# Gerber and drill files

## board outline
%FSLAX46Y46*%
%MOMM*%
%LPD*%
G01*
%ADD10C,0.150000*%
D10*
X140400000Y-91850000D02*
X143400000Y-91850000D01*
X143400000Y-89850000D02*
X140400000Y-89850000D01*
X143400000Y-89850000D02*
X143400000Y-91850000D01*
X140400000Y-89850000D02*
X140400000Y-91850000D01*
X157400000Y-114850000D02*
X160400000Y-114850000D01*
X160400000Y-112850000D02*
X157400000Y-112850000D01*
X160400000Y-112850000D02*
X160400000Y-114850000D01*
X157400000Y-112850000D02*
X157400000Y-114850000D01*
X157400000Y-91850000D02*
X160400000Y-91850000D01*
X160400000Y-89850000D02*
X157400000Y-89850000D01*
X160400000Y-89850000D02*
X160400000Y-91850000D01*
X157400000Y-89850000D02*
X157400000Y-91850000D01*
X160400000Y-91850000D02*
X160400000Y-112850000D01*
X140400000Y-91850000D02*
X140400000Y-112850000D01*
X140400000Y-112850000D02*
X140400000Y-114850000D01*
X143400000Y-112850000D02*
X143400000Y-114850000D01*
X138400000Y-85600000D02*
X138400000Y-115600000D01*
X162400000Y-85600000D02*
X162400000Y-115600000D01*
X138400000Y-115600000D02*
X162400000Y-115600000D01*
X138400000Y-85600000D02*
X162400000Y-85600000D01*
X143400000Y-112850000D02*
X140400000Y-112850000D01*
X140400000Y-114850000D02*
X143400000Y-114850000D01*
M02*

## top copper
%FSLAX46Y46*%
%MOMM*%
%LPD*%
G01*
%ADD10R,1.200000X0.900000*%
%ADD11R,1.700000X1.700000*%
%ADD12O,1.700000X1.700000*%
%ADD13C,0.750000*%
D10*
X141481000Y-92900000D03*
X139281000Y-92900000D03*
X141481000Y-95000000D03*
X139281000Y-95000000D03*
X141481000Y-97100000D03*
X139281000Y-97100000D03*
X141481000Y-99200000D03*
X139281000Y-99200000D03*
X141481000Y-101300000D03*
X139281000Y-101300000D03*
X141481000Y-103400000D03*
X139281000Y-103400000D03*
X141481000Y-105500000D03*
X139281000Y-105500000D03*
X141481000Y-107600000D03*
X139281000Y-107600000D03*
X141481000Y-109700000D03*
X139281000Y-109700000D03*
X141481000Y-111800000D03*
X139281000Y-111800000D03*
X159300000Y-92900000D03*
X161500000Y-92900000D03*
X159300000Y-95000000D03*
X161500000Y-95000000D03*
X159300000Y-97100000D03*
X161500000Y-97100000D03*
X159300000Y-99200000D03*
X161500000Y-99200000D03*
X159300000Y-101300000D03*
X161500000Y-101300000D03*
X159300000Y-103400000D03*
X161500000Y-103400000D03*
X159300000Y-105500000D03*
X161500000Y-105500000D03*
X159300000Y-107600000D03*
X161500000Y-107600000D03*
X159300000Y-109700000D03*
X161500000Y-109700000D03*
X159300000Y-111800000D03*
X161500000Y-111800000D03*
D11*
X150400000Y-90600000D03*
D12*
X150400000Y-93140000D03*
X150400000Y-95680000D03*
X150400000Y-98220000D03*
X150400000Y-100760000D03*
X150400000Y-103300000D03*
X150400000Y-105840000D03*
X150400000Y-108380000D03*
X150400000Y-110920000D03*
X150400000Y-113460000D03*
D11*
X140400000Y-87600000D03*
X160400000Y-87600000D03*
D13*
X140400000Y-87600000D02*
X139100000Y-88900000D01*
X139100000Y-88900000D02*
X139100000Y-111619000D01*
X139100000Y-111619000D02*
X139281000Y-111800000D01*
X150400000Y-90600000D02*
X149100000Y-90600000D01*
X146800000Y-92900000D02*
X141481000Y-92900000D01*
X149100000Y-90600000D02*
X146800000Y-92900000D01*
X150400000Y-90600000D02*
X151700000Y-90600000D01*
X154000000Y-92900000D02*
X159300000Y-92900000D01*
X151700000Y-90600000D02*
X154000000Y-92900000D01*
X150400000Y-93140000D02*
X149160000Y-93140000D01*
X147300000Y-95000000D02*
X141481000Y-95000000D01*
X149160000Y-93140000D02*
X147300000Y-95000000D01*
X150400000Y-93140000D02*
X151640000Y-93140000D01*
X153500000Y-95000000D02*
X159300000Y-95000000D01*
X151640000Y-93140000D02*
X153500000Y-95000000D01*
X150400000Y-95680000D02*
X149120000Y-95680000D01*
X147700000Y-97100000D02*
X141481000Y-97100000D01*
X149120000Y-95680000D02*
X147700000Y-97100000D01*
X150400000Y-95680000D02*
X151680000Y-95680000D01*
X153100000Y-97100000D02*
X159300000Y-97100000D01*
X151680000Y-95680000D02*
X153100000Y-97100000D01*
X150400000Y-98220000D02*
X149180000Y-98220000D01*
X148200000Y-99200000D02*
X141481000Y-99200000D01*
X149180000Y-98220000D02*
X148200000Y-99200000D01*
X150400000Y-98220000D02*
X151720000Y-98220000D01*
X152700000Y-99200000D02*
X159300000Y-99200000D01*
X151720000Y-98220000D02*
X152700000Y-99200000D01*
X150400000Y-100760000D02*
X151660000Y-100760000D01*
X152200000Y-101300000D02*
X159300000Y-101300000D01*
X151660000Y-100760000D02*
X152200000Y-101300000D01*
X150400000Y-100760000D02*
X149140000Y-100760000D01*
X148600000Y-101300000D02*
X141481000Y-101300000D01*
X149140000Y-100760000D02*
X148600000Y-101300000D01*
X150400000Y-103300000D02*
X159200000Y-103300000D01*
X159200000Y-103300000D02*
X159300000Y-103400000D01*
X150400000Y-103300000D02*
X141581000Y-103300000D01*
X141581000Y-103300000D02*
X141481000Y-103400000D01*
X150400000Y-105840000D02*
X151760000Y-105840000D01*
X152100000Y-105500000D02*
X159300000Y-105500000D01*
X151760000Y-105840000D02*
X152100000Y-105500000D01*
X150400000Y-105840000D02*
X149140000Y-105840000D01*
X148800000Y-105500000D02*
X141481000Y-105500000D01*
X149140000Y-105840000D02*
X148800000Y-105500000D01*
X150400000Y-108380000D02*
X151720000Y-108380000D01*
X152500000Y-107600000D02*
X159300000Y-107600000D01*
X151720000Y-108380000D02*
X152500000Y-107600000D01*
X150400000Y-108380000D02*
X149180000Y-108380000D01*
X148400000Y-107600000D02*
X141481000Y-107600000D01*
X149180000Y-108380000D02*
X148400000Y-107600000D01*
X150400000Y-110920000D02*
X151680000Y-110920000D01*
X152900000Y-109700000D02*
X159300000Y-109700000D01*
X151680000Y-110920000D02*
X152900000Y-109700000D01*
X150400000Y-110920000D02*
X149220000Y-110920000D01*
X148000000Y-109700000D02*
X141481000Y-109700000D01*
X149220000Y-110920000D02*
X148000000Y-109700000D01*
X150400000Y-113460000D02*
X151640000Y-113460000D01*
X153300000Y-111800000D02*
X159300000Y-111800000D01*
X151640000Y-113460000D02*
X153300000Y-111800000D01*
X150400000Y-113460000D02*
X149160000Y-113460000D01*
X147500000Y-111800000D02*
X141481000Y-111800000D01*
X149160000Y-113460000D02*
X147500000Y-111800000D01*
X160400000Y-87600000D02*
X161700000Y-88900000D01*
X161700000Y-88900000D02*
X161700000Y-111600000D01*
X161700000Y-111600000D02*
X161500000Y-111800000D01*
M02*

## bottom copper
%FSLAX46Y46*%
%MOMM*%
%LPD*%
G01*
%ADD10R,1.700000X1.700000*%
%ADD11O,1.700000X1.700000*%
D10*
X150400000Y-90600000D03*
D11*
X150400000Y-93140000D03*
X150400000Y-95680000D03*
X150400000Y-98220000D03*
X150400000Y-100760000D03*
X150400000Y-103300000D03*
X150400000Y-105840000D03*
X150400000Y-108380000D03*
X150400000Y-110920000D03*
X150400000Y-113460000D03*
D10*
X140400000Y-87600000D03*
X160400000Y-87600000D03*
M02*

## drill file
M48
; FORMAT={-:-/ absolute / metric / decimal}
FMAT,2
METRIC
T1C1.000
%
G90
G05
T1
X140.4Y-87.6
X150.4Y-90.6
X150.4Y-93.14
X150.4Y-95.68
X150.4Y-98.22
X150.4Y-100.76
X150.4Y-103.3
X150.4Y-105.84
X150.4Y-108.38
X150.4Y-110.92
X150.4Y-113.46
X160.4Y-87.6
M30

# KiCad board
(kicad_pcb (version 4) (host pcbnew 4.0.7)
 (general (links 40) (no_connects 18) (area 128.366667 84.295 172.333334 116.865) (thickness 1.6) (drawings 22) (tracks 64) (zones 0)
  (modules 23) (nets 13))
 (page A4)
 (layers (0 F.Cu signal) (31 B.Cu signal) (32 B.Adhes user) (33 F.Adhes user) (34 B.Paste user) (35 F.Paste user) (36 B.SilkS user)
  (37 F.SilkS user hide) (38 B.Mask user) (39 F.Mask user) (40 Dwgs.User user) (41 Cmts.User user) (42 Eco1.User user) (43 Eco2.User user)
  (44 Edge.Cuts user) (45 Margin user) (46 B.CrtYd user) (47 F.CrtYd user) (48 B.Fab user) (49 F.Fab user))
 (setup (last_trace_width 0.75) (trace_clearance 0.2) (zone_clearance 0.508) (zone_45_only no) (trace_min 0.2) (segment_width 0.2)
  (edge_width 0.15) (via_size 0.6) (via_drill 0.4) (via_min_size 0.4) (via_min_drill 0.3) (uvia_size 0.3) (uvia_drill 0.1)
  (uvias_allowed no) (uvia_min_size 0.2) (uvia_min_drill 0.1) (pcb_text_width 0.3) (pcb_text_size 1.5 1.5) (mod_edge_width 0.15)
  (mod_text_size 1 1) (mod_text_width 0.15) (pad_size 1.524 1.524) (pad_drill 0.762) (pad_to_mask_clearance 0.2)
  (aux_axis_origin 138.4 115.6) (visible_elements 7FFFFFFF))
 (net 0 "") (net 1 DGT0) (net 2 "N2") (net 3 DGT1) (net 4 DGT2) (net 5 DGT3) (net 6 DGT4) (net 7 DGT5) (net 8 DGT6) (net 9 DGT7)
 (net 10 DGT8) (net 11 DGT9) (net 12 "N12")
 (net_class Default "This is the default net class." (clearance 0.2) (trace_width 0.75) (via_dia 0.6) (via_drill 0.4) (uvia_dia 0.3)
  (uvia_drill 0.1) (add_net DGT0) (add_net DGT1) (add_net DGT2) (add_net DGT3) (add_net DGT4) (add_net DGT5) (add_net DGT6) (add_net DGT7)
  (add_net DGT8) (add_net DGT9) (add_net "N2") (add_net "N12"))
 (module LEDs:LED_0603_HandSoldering (layer F.Cu) (at 140.381 92.9 180)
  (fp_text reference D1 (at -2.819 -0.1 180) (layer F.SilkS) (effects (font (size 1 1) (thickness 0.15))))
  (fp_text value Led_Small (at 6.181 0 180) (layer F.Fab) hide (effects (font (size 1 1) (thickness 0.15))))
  (pad 1 smd rect (at -1.1 0 180) (size 1.2 0.9) (layers F.Cu F.Paste F.Mask) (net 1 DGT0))
  (pad 2 smd rect (at 1.1 0 180) (size 1.2 0.9) (layers F.Cu F.Paste F.Mask) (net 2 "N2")))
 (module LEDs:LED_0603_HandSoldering (layer F.Cu) (at 140.381 95 180)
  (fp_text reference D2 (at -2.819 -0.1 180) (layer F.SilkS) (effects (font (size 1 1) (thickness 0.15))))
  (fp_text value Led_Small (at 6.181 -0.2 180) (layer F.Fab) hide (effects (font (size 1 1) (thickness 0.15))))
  (pad 1 smd rect (at -1.1 0 180) (size 1.2 0.9) (layers F.Cu F.Paste F.Mask) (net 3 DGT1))
  (pad 2 smd rect (at 1.1 0 180) (size 1.2 0.9) (layers F.Cu F.Paste F.Mask) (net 2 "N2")))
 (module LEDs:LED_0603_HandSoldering (layer F.Cu) (at 140.381 97.1 180)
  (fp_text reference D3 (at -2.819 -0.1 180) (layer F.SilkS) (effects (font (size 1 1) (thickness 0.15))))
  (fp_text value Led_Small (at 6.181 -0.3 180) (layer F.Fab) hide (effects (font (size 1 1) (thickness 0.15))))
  (pad 1 smd rect (at -1.1 0 180) (size 1.2 0.9) (layers F.Cu F.Paste F.Mask) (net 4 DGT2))
  (pad 2 smd rect (at 1.1 0 180) (size 1.2 0.9) (layers F.Cu F.Paste F.Mask) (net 2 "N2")))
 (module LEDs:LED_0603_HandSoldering (layer F.Cu) (at 140.381 99.2 180)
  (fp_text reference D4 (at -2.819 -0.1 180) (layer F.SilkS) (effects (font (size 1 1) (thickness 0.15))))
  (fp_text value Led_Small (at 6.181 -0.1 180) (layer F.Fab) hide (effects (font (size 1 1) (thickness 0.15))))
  (pad 1 smd rect (at -1.1 0 180) (size 1.2 0.9) (layers F.Cu F.Paste F.Mask) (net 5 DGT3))
  (pad 2 smd rect (at 1.1 0 180) (size 1.2 0.9) (layers F.Cu F.Paste F.Mask) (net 2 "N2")))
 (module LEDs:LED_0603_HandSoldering (layer F.Cu) (at 140.381 101.3 180)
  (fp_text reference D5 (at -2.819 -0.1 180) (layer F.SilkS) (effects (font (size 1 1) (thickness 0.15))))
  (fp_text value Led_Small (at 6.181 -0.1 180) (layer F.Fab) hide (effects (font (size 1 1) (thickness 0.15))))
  (pad 1 smd rect (at -1.1 0 180) (size 1.2 0.9) (layers F.Cu F.Paste F.Mask) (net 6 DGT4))
  (pad 2 smd rect (at 1.1 0 180) (size 1.2 0.9) (layers F.Cu F.Paste F.Mask) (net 2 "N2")))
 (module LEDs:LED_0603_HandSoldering (layer F.Cu) (at 140.381 103.4 180)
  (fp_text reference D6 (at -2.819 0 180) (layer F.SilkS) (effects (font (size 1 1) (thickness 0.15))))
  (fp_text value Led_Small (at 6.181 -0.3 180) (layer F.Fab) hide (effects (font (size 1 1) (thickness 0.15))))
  (pad 1 smd rect (at -1.1 0 180) (size 1.2 0.9) (layers F.Cu F.Paste F.Mask) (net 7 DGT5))
  (pad 2 smd rect (at 1.1 0 180) (size 1.2 0.9) (layers F.Cu F.Paste F.Mask) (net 2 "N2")))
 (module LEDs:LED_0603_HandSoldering (layer F.Cu) (at 140.381 105.5 180)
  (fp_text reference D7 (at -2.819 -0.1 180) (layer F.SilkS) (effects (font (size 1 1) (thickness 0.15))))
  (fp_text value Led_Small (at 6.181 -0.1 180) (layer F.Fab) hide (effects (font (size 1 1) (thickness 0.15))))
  (pad 1 smd rect (at -1.1 0 180) (size 1.2 0.9) (layers F.Cu F.Paste F.Mask) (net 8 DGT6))
  (pad 2 smd rect (at 1.1 0 180) (size 1.2 0.9) (layers F.Cu F.Paste F.Mask) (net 2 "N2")))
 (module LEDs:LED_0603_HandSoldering (layer F.Cu) (at 140.381 107.6 180)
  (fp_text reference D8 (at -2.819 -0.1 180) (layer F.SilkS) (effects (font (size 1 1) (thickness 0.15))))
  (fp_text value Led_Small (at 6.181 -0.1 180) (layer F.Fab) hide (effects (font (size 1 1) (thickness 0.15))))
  (pad 1 smd rect (at -1.1 0 180) (size 1.2 0.9) (layers F.Cu F.Paste F.Mask) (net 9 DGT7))
  (pad 2 smd rect (at 1.1 0 180) (size 1.2 0.9) (layers F.Cu F.Paste F.Mask) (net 2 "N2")))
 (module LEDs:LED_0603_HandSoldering (layer F.Cu) (at 140.381 109.7 180)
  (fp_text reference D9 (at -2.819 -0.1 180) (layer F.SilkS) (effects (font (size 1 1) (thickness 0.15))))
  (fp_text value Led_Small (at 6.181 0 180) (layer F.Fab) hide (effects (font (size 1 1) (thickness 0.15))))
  (pad 1 smd rect (at -1.1 0 180) (size 1.2 0.9) (layers F.Cu F.Paste F.Mask) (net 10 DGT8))
  (pad 2 smd rect (at 1.1 0 180) (size 1.2 0.9) (layers F.Cu F.Paste F.Mask) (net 2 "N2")))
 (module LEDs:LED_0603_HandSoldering (layer F.Cu) (at 140.381 111.8 180)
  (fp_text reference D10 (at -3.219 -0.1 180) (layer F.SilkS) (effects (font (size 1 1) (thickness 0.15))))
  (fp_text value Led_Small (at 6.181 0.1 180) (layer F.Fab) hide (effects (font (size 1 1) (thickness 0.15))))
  (pad 1 smd rect (at -1.1 0 180) (size 1.2 0.9) (layers F.Cu F.Paste F.Mask) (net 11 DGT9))
  (pad 2 smd rect (at 1.1 0 180) (size 1.2 0.9) (layers F.Cu F.Paste F.Mask) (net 2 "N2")))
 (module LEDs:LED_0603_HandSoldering (layer F.Cu) (at 160.4 92.9)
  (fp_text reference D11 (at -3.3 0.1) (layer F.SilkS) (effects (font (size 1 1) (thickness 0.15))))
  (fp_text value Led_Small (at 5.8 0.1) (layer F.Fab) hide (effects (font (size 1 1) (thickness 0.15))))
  (pad 1 smd rect (at -1.1 0) (size 1.2 0.9) (layers F.Cu F.Paste F.Mask) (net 1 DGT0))
  (pad 2 smd rect (at 1.1 0) (size 1.2 0.9) (layers F.Cu F.Paste F.Mask) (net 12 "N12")))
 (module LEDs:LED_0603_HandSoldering (layer F.Cu) (at 160.4 95)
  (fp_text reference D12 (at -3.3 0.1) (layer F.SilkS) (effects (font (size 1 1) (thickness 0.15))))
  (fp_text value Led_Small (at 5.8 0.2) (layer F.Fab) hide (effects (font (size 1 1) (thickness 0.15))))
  (pad 1 smd rect (at -1.1 0) (size 1.2 0.9) (layers F.Cu F.Paste F.Mask) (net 3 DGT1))
  (pad 2 smd rect (at 1.1 0) (size 1.2 0.9) (layers F.Cu F.Paste F.Mask) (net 12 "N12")))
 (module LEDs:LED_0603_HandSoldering (layer F.Cu) (at 160.4 97.1)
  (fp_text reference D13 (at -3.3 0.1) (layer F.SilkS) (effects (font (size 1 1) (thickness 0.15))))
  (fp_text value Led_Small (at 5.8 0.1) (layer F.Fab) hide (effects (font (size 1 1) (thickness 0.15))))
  (pad 1 smd rect (at -1.1 0) (size 1.2 0.9) (layers F.Cu F.Paste F.Mask) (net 4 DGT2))
  (pad 2 smd rect (at 1.1 0) (size 1.2 0.9) (layers F.Cu F.Paste F.Mask) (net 12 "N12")))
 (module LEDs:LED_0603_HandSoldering (layer F.Cu) (at 160.4 99.2)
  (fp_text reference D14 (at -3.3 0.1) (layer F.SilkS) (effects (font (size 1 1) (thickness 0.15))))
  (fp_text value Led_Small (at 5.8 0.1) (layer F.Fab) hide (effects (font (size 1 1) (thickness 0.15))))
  (pad 1 smd rect (at -1.1 0) (size 1.2 0.9) (layers F.Cu F.Paste F.Mask) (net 5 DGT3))
  (pad 2 smd rect (at 1.1 0) (size 1.2 0.9) (layers F.Cu F.Paste F.Mask) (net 12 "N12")))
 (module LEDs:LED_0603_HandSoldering (layer F.Cu) (at 160.4 101.3)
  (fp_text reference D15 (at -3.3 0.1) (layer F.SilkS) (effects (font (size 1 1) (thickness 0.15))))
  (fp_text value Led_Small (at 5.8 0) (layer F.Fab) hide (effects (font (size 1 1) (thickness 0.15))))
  (pad 1 smd rect (at -1.1 0) (size 1.2 0.9) (layers F.Cu F.Paste F.Mask) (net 6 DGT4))
  (pad 2 smd rect (at 1.1 0) (size 1.2 0.9) (layers F.Cu F.Paste F.Mask) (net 12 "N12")))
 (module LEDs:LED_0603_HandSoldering (layer F.Cu) (at 160.4 103.4)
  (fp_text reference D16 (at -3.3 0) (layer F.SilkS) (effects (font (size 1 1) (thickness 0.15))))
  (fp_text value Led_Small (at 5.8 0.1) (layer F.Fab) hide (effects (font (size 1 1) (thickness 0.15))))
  (pad 1 smd rect (at -1.1 0) (size 1.2 0.9) (layers F.Cu F.Paste F.Mask) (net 7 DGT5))
  (pad 2 smd rect (at 1.1 0) (size 1.2 0.9) (layers F.Cu F.Paste F.Mask) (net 12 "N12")))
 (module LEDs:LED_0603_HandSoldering (layer F.Cu) (at 160.4 105.5)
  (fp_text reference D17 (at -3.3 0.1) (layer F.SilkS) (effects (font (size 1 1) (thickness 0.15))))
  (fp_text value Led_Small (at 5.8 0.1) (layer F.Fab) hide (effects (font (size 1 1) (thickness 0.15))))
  (pad 1 smd rect (at -1.1 0) (size 1.2 0.9) (layers F.Cu F.Paste F.Mask) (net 8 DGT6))
  (pad 2 smd rect (at 1.1 0) (size 1.2 0.9) (layers F.Cu F.Paste F.Mask) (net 12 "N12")))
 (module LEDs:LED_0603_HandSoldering (layer F.Cu) (at 160.4 107.6)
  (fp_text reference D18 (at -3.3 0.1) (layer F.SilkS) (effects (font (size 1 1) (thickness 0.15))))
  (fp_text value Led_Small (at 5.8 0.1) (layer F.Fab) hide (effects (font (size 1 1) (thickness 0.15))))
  (pad 1 smd rect (at -1.1 0) (size 1.2 0.9) (layers F.Cu F.Paste F.Mask) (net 9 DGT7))
  (pad 2 smd rect (at 1.1 0) (size 1.2 0.9) (layers F.Cu F.Paste F.Mask) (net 12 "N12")))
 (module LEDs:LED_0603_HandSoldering (layer F.Cu) (at 160.4 109.7)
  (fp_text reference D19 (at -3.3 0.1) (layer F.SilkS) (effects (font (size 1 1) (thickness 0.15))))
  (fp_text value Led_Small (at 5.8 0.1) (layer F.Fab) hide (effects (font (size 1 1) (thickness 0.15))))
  (pad 1 smd rect (at -1.1 0) (size 1.2 0.9) (layers F.Cu F.Paste F.Mask) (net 10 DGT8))
  (pad 2 smd rect (at 1.1 0) (size 1.2 0.9) (layers F.Cu F.Paste F.Mask) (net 12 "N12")))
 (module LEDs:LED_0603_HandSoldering (layer F.Cu) (at 160.4 111.8)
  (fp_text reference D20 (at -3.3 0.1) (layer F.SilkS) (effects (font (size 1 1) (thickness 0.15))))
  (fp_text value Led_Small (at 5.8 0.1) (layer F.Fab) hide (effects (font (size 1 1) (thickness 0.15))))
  (pad 1 smd rect (at -1.1 0) (size 1.2 0.9) (layers F.Cu F.Paste F.Mask) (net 11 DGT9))
  (pad 2 smd rect (at 1.1 0) (size 1.2 0.9) (layers F.Cu F.Paste F.Mask) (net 12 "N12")))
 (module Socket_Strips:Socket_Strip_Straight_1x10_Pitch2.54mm (layer F.Cu) (at 150.4 90.6)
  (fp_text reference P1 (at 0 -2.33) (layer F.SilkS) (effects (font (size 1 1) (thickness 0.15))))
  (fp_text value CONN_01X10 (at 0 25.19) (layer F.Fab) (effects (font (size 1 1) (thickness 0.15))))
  (pad 1 thru_hole rect (at 0 0) (size 1.7 1.7) (drill 1) (layers *.Cu *.Mask) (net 1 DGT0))
  (pad 2 thru_hole oval (at 0 2.54) (size 1.7 1.7) (drill 1) (layers *.Cu *.Mask) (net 3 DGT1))
  (pad 3 thru_hole oval (at 0 5.08) (size 1.7 1.7) (drill 1) (layers *.Cu *.Mask) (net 4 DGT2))
  (pad 4 thru_hole oval (at 0 7.62) (size 1.7 1.7) (drill 1) (layers *.Cu *.Mask) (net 5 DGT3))
  (pad 5 thru_hole oval (at 0 10.16) (size 1.7 1.7) (drill 1) (layers *.Cu *.Mask) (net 6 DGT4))
  (pad 6 thru_hole oval (at 0 12.7) (size 1.7 1.7) (drill 1) (layers *.Cu *.Mask) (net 7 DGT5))
  (pad 7 thru_hole oval (at 0 15.24) (size 1.7 1.7) (drill 1) (layers *.Cu *.Mask) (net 8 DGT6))
  (pad 8 thru_hole oval (at 0 17.78) (size 1.7 1.7) (drill 1) (layers *.Cu *.Mask) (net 9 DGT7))
  (pad 9 thru_hole oval (at 0 20.32) (size 1.7 1.7) (drill 1) (layers *.Cu *.Mask) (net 10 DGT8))
  (pad 10 thru_hole oval (at 0 22.86) (size 1.7 1.7) (drill 1) (layers *.Cu *.Mask) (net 11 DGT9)))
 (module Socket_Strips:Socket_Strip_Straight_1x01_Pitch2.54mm (layer F.Cu) (at 140.4 87.6)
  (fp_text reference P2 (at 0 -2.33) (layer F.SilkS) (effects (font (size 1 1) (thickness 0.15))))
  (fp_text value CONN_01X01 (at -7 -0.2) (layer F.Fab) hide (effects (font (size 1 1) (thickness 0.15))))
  (pad 1 thru_hole rect (at 0 0) (size 1.7 1.7) (drill 1) (layers *.Cu *.Mask) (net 2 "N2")))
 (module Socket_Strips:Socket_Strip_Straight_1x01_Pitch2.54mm (layer F.Cu) (at 160.4 87.6)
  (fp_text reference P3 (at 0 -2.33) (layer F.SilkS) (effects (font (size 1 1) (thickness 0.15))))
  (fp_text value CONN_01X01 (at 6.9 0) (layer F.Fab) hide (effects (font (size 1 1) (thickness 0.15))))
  (pad 1 thru_hole rect (at 0 0) (size 1.7 1.7) (drill 1) (layers *.Cu *.Mask) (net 12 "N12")))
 (gr_line (start 140.4 91.85) (end 143.4 91.85) (angle 90) (layer Edge.Cuts) (width 0.15))
 (gr_line (start 143.4 89.85) (end 140.4 89.85) (angle 90) (layer Edge.Cuts) (width 0.15))
 (gr_line (start 143.4 89.85) (end 143.4 91.85) (angle 90) (layer Edge.Cuts) (width 0.15))
 (gr_line (start 140.4 89.85) (end 140.4 91.85) (angle 90) (layer Edge.Cuts) (width 0.15))
 (gr_line (start 157.4 114.85) (end 160.4 114.85) (angle 90) (layer Edge.Cuts) (width 0.15))
 (gr_line (start 160.4 112.85) (end 157.4 112.85) (angle 90) (layer Edge.Cuts) (width 0.15))
 (gr_line (start 160.4 112.85) (end 160.4 114.85) (angle 90) (layer Edge.Cuts) (width 0.15))
 (gr_line (start 157.4 112.85) (end 157.4 114.85) (angle 90) (layer Edge.Cuts) (width 0.15))
 (gr_line (start 157.4 91.85) (end 160.4 91.85) (angle 90) (layer Edge.Cuts) (width 0.15))
 (gr_line (start 160.4 89.85) (end 157.4 89.85) (angle 90) (layer Edge.Cuts) (width 0.15))
 (gr_line (start 160.4 89.85) (end 160.4 91.85) (angle 90) (layer Edge.Cuts) (width 0.15))
 (gr_line (start 157.4 89.85) (end 157.4 91.85) (angle 90) (layer Edge.Cuts) (width 0.15))
 (gr_line (start 160.4 91.85) (end 160.4 112.85) (angle 90) (layer Edge.Cuts) (width 0.15))
 (gr_line (start 140.4 91.85) (end 140.4 112.85) (angle 90) (layer Edge.Cuts) (width 0.15))
 (gr_line (start 140.4 112.85) (end 140.4 114.85) (angle 90) (layer Edge.Cuts) (width 0.15))
 (gr_line (start 143.4 112.85) (end 143.4 114.85) (angle 90) (layer Edge.Cuts) (width 0.15))
 (gr_line (start 138.4 85.6) (end 138.4 115.6) (angle 90) (layer Edge.Cuts) (width 0.15))
 (gr_line (start 162.4 85.6) (end 162.4 115.6) (angle 90) (layer Edge.Cuts) (width 0.15))
 (gr_line (start 138.4 115.6) (end 162.4 115.6) (angle 90) (layer Edge.Cuts) (width 0.15))
 (gr_line (start 138.4 85.6) (end 162.4 85.6) (angle 90) (layer Edge.Cuts) (width 0.15))
 (gr_line (start 143.4 112.85) (end 140.4 112.85) (angle 90) (layer Edge.Cuts) (width 0.15))
 (gr_line (start 140.4 114.85) (end 143.4 114.85) (angle 90) (layer Edge.Cuts) (width 0.15))
 (segment (start 140.4 87.6) (end 139.1 88.9) (width 0.75) (layer F.Cu) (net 2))
 (segment (start 139.1 88.9) (end 139.1 111.619) (width 0.75) (layer F.Cu) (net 2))
 (segment (start 139.1 111.619) (end 139.281 111.8) (width 0.75) (layer F.Cu) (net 2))
 (segment (start 150.4 90.6) (end 149.1 90.6) (width 0.75) (layer F.Cu) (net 1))
 (segment (start 146.8 92.9) (end 141.481 92.9) (width 0.75) (layer F.Cu) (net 1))
 (segment (start 149.1 90.6) (end 146.8 92.9) (width 0.75) (layer F.Cu) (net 1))
 (segment (start 150.4 90.6) (end 151.7 90.6) (width 0.75) (layer F.Cu) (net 1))
 (segment (start 154 92.9) (end 159.3 92.9) (width 0.75) (layer F.Cu) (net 1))
 (segment (start 151.7 90.6) (end 154 92.9) (width 0.75) (layer F.Cu) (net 1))
 (segment (start 150.4 93.14) (end 149.16 93.14) (width 0.75) (layer F.Cu) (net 3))
 (segment (start 147.3 95) (end 141.481 95) (width 0.75) (layer F.Cu) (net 3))
 (segment (start 149.16 93.14) (end 147.3 95) (width 0.75) (layer F.Cu) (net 3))
 (segment (start 150.4 93.14) (end 151.64 93.14) (width 0.75) (layer F.Cu) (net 3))
 (segment (start 153.5 95) (end 159.3 95) (width 0.75) (layer F.Cu) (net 3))
 (segment (start 151.64 93.14) (end 153.5 95) (width 0.75) (layer F.Cu) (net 3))
 (segment (start 150.4 95.68) (end 149.12 95.68) (width 0.75) (layer F.Cu) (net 4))
 (segment (start 147.7 97.1) (end 141.481 97.1) (width 0.75) (layer F.Cu) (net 4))
 (segment (start 149.12 95.68) (end 147.7 97.1) (width 0.75) (layer F.Cu) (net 4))
 (segment (start 150.4 95.68) (end 151.68 95.68) (width 0.75) (layer F.Cu) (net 4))
 (segment (start 153.1 97.1) (end 159.3 97.1) (width 0.75) (layer F.Cu) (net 4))
 (segment (start 151.68 95.68) (end 153.1 97.1) (width 0.75) (layer F.Cu) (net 4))
 (segment (start 150.4 98.22) (end 149.18 98.22) (width 0.75) (layer F.Cu) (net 5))
 (segment (start 148.2 99.2) (end 141.481 99.2) (width 0.75) (layer F.Cu) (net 5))
 (segment (start 149.18 98.22) (end 148.2 99.2) (width 0.75) (layer F.Cu) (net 5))
 (segment (start 150.4 98.22) (end 151.72 98.22) (width 0.75) (layer F.Cu) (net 5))
 (segment (start 152.7 99.2) (end 159.3 99.2) (width 0.75) (layer F.Cu) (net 5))
 (segment (start 151.72 98.22) (end 152.7 99.2) (width 0.75) (layer F.Cu) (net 5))
 (segment (start 150.4 100.76) (end 151.66 100.76) (width 0.75) (layer F.Cu) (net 6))
 (segment (start 152.2 101.3) (end 159.3 101.3) (width 0.75) (layer F.Cu) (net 6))
 (segment (start 151.66 100.76) (end 152.2 101.3) (width 0.75) (layer F.Cu) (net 6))
 (segment (start 150.4 100.76) (end 149.14 100.76) (width 0.75) (layer F.Cu) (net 6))
 (segment (start 148.6 101.3) (end 141.481 101.3) (width 0.75) (layer F.Cu) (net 6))
 (segment (start 149.14 100.76) (end 148.6 101.3) (width 0.75) (layer F.Cu) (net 6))
 (segment (start 150.4 103.3) (end 159.2 103.3) (width 0.75) (layer F.Cu) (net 7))
 (segment (start 159.2 103.3) (end 159.3 103.4) (width 0.75) (layer F.Cu) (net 7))
 (segment (start 150.4 103.3) (end 141.581 103.3) (width 0.75) (layer F.Cu) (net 7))
 (segment (start 141.581 103.3) (end 141.481 103.4) (width 0.75) (layer F.Cu) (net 7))
 (segment (start 150.4 105.84) (end 151.76 105.84) (width 0.75) (layer F.Cu) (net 8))
 (segment (start 152.1 105.5) (end 159.3 105.5) (width 0.75) (layer F.Cu) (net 8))
 (segment (start 151.76 105.84) (end 152.1 105.5) (width 0.75) (layer F.Cu) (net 8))
 (segment (start 150.4 105.84) (end 149.14 105.84) (width 0.75) (layer F.Cu) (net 8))
 (segment (start 148.8 105.5) (end 141.481 105.5) (width 0.75) (layer F.Cu) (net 8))
 (segment (start 149.14 105.84) (end 148.8 105.5) (width 0.75) (layer F.Cu) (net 8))
 (segment (start 150.4 108.38) (end 151.72 108.38) (width 0.75) (layer F.Cu) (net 9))
 (segment (start 152.5 107.6) (end 159.3 107.6) (width 0.75) (layer F.Cu) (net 9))
 (segment (start 151.72 108.38) (end 152.5 107.6) (width 0.75) (layer F.Cu) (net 9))
 (segment (start 150.4 108.38) (end 149.18 108.38) (width 0.75) (layer F.Cu) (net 9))
 (segment (start 148.4 107.6) (end 141.481 107.6) (width 0.75) (layer F.Cu) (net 9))
 (segment (start 149.18 108.38) (end 148.4 107.6) (width 0.75) (layer F.Cu) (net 9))
 (segment (start 150.4 110.92) (end 151.68 110.92) (width 0.75) (layer F.Cu) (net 10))
 (segment (start 152.9 109.7) (end 159.3 109.7) (width 0.75) (layer F.Cu) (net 10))
 (segment (start 151.68 110.92) (end 152.9 109.7) (width 0.75) (layer F.Cu) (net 10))
 (segment (start 150.4 110.92) (end 149.22 110.92) (width 0.75) (layer F.Cu) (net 10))
 (segment (start 148 109.7) (end 141.481 109.7) (width 0.75) (layer F.Cu) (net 10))
 (segment (start 149.22 110.92) (end 148 109.7) (width 0.75) (layer F.Cu) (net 10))
 (segment (start 150.4 113.46) (end 151.64 113.46) (width 0.75) (layer F.Cu) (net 11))
 (segment (start 153.3 111.8) (end 159.3 111.8) (width 0.75) (layer F.Cu) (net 11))
 (segment (start 151.64 113.46) (end 153.3 111.8) (width 0.75) (layer F.Cu) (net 11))
 (segment (start 150.4 113.46) (end 149.16 113.46) (width 0.75) (layer F.Cu) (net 11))
 (segment (start 147.5 111.8) (end 141.481 111.8) (width 0.75) (layer F.Cu) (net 11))
 (segment (start 149.16 113.46) (end 147.5 111.8) (width 0.75) (layer F.Cu) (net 11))
 (segment (start 160.4 87.6) (end 161.7 88.9) (width 0.75) (layer F.Cu) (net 12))
 (segment (start 161.7 88.9) (end 161.7 111.6) (width 0.75) (layer F.Cu) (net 12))
 (segment (start 161.7 111.6) (end 161.5 111.8) (width 0.75) (layer F.Cu) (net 12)))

